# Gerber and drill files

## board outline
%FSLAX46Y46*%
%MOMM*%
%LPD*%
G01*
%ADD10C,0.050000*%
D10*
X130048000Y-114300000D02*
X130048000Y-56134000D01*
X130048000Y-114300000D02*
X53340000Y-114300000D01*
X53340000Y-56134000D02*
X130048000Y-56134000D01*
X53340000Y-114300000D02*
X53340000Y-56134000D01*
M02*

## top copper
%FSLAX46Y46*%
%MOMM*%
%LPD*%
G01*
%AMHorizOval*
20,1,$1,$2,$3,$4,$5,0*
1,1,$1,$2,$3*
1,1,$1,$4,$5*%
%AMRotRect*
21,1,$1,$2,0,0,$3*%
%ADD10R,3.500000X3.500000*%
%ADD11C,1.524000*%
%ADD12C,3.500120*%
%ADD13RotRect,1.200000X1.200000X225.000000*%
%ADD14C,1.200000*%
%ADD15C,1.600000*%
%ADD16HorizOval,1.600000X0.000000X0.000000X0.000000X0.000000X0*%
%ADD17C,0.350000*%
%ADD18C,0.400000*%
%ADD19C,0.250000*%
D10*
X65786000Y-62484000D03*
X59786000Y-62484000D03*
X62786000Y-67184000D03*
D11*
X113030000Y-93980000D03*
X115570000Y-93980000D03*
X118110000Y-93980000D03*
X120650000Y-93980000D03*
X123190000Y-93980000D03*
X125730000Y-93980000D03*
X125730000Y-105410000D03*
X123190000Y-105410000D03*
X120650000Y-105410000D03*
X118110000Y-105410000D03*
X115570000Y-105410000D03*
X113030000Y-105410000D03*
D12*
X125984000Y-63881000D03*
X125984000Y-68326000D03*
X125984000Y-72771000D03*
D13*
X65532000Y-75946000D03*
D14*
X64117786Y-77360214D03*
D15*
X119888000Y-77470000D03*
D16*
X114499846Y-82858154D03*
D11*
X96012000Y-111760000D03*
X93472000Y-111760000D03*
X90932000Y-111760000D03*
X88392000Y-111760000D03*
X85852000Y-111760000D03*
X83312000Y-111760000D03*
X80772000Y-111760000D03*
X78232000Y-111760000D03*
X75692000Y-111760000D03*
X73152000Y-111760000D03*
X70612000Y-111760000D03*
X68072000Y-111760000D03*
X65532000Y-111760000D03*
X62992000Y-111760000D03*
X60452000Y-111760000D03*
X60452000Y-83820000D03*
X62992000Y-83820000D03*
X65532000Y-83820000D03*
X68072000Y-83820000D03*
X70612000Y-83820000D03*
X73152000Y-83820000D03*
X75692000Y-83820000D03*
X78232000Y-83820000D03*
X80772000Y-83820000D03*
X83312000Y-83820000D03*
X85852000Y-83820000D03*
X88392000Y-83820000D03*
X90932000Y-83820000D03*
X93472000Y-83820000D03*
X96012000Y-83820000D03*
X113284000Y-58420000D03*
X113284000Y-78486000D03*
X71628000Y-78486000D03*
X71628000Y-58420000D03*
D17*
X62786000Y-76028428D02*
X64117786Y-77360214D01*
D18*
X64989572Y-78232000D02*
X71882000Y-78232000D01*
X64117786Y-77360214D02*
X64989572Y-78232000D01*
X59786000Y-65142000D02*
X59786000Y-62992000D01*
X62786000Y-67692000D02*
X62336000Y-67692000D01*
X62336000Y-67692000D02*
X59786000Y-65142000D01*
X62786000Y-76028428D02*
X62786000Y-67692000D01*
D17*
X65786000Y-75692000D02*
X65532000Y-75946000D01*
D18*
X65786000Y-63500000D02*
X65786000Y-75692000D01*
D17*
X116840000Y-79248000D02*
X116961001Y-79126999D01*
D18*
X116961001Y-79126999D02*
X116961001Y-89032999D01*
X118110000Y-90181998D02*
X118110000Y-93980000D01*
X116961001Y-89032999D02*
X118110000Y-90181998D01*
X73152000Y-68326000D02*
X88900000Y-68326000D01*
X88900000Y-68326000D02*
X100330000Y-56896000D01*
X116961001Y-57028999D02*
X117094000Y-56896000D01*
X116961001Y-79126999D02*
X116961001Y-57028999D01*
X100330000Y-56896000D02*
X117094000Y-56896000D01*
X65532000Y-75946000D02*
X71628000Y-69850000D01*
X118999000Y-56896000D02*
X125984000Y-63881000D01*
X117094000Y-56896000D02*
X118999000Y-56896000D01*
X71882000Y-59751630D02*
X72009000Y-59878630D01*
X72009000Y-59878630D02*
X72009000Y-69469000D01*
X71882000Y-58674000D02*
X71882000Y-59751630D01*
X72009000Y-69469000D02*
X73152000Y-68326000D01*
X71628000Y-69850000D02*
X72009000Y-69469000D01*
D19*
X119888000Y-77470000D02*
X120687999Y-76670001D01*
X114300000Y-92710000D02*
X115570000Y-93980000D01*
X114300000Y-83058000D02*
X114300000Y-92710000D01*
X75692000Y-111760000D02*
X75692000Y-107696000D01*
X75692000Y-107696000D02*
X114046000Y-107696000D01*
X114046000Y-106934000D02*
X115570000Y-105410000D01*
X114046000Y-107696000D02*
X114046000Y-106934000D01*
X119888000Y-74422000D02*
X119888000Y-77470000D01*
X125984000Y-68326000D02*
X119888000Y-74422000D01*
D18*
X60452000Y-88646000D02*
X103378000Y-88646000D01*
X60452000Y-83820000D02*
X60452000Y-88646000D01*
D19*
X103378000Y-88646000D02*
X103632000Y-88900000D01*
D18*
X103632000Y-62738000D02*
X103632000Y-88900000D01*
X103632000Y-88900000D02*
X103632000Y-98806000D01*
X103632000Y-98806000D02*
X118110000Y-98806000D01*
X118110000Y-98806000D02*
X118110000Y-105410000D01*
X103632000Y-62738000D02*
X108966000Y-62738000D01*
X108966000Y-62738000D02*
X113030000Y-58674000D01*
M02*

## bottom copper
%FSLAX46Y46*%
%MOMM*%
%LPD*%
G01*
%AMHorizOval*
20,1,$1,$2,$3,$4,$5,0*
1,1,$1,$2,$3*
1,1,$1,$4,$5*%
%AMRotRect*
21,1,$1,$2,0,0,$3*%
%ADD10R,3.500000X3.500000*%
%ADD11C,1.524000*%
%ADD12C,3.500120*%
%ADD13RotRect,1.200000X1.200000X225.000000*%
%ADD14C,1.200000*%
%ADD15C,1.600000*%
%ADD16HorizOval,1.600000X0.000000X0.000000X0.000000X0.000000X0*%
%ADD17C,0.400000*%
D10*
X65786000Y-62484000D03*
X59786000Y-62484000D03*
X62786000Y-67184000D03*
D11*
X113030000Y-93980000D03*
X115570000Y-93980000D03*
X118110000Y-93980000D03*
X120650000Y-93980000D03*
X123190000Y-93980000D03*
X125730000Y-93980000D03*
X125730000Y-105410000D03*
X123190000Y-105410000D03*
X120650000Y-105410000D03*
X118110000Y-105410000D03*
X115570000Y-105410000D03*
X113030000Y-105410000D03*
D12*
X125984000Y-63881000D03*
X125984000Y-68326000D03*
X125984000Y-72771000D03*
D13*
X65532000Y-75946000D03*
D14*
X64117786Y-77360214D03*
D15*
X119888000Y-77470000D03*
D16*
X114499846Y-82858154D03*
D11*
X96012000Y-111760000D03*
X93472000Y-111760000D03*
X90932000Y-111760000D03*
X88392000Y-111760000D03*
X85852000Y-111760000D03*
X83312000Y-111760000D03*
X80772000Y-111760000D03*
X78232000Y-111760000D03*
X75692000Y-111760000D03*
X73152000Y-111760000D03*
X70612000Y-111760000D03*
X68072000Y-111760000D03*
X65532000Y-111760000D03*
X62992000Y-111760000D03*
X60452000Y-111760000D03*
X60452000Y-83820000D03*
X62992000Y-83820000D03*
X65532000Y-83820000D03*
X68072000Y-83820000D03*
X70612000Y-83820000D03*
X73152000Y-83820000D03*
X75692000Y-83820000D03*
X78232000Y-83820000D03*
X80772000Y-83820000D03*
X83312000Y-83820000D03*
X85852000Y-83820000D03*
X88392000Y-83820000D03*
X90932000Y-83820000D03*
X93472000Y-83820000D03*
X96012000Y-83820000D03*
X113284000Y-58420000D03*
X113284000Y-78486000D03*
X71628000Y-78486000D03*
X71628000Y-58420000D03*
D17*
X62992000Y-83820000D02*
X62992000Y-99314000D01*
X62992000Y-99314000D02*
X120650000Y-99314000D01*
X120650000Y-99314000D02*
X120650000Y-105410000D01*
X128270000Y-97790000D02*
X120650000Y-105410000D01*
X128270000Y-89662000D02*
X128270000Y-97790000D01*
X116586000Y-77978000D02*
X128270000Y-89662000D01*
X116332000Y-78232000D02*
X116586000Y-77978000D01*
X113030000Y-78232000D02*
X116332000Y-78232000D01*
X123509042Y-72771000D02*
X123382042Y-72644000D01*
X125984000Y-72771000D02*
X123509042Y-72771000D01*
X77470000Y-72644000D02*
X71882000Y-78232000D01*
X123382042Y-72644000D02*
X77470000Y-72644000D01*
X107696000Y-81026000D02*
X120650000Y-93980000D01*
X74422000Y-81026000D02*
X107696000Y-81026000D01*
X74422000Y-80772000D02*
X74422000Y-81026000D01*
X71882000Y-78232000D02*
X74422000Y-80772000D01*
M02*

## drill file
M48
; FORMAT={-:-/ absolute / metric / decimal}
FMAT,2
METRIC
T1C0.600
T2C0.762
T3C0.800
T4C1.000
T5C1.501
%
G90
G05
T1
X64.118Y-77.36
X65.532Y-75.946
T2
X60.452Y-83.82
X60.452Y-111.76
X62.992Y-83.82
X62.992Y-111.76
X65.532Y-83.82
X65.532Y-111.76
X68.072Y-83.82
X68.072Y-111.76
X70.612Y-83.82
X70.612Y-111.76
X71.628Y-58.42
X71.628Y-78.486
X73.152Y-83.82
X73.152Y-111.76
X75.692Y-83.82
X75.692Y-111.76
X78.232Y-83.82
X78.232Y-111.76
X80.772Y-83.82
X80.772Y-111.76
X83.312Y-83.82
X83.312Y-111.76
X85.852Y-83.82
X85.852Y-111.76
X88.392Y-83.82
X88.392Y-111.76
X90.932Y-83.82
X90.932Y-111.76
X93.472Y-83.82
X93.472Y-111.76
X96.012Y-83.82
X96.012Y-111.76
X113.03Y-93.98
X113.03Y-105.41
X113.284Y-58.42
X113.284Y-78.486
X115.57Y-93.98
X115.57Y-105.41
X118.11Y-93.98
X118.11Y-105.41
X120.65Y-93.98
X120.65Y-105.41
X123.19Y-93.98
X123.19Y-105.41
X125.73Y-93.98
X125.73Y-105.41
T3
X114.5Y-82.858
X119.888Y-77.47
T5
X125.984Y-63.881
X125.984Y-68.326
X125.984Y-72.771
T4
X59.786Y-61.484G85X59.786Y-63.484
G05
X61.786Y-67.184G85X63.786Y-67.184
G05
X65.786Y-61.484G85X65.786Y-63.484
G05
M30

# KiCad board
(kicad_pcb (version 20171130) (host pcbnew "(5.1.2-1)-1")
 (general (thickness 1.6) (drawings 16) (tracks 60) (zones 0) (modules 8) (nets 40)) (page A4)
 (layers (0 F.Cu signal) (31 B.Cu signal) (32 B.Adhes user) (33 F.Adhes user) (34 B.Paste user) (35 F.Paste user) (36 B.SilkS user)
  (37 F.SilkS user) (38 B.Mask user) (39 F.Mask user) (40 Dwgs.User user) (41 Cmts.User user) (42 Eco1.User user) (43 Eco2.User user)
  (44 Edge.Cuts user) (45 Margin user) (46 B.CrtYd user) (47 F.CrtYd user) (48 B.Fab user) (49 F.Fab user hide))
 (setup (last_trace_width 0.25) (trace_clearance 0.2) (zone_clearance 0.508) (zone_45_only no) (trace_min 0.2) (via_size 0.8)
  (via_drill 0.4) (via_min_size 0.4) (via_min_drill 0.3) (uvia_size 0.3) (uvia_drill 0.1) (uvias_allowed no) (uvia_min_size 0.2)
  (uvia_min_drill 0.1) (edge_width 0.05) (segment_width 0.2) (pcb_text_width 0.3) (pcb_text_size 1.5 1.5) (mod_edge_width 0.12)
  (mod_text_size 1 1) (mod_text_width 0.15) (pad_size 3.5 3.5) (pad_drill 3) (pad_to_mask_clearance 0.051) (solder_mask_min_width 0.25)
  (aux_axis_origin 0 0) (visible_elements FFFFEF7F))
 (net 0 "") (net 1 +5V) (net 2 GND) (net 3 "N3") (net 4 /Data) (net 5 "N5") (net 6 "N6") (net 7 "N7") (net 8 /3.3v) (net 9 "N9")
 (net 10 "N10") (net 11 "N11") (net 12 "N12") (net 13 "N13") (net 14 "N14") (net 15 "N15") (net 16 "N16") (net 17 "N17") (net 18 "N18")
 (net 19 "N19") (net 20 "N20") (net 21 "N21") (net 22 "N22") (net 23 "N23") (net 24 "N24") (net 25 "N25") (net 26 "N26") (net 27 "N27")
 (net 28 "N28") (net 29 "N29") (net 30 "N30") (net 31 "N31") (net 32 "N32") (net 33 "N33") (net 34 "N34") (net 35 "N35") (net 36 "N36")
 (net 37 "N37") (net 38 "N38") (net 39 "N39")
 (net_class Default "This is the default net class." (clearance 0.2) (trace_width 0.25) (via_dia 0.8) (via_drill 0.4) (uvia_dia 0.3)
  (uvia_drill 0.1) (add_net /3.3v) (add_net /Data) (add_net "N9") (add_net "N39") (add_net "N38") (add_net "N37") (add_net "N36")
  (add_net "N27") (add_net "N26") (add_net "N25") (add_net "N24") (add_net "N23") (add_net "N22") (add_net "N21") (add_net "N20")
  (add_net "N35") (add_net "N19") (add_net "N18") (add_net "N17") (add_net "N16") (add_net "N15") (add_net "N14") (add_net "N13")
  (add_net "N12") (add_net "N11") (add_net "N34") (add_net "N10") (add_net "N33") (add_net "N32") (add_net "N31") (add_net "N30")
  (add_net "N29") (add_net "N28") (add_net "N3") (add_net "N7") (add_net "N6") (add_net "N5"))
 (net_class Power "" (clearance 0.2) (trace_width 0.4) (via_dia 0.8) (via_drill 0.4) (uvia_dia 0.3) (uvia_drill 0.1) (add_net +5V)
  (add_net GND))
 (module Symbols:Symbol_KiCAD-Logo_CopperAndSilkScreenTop (layer F.Cu) (at 119.126 88.392)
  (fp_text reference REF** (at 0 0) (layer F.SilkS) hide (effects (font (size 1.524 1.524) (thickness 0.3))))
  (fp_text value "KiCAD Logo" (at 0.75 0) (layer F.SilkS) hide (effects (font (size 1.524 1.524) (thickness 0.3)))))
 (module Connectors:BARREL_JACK (layer F.Cu) (at 65.786 62.484)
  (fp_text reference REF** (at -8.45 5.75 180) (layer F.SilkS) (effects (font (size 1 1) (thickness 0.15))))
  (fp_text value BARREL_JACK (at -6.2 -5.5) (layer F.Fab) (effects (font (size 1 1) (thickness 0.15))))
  (pad 1 thru_hole rect (at 0 0) (size 3.5 3.5) (drill oval 1 3) (layers *.Cu *.Mask) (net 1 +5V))
  (pad 2 thru_hole rect (at -6 0) (size 3.5 3.5) (drill oval 1 3) (layers *.Cu *.Mask) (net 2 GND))
  (pad 3 thru_hole rect (at -3 4.7) (size 3.5 3.5) (drill oval 3 1) (layers *.Cu *.Mask) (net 2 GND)))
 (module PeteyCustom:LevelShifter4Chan (layer F.Cu) (at 118.11 100.33 90)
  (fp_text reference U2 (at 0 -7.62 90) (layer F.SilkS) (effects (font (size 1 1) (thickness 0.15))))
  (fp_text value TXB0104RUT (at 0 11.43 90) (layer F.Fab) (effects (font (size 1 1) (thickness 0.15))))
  (pad 12 thru_hole circle (at 6.35 -5.08 90) (size 1.524 1.524) (drill 0.762) (layers *.Cu *.Mask) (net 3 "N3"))
  (pad 11 thru_hole circle (at 6.35 -2.54 90) (size 1.524 1.524) (drill 0.762) (layers *.Cu *.Mask) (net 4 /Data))
  (pad 10 thru_hole circle (at 6.35 0 90) (size 1.524 1.524) (drill 0.762) (layers *.Cu *.Mask) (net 1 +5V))
  (pad 9 thru_hole circle (at 6.35 2.54 90) (size 1.524 1.524) (drill 0.762) (layers *.Cu *.Mask) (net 2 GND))
  (pad 8 thru_hole circle (at 6.35 5.08 90) (size 1.524 1.524) (drill 0.762) (layers *.Cu *.Mask) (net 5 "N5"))
  (pad 7 thru_hole circle (at 6.35 7.62 90) (size 1.524 1.524) (drill 0.762) (layers *.Cu *.Mask) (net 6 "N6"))
  (pad 6 thru_hole circle (at -5.08 7.62 90) (size 1.524 1.524) (drill 0.762) (layers *.Cu *.Mask))
  (pad 5 thru_hole circle (at -5.08 5.08 90) (size 1.524 1.524) (drill 0.762) (layers *.Cu *.Mask) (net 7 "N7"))
  (pad 4 thru_hole circle (at -5.08 2.54 90) (size 1.524 1.524) (drill 0.762) (layers *.Cu *.Mask) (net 2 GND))
  (pad 3 thru_hole circle (at -5.08 0 90) (size 1.524 1.524) (drill 0.762) (layers *.Cu *.Mask) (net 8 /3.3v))
  (pad 2 thru_hole circle (at -5.08 -2.54 90) (size 1.524 1.524) (drill 0.762) (layers *.Cu *.Mask) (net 4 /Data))
  (pad 1 thru_hole circle (at -5.08 -5.08 90) (size 1.524 1.524) (drill 0.762) (layers *.Cu *.Mask)))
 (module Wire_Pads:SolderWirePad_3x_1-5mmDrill (layer F.Cu) (at 125.984 68.326 270)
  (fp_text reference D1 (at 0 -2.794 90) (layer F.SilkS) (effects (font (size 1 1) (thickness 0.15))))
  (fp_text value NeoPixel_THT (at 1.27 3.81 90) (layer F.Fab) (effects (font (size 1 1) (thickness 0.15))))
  (pad 1 thru_hole circle (at -4.445 0 270) (size 3.50012 3.50012) (drill 1.50114) (layers *.Cu *.Mask) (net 1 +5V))
  (pad 2 thru_hole circle (at 0 0 270) (size 3.50012 3.50012) (drill 1.50114) (layers *.Cu *.Mask) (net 4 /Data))
  (pad 3 thru_hole circle (at 4.445 0 270) (size 3.50012 3.50012) (drill 1.50114) (layers *.Cu *.Mask) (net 2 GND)))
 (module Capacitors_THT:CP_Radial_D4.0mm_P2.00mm (layer F.Cu) (at 65.532 75.946 225)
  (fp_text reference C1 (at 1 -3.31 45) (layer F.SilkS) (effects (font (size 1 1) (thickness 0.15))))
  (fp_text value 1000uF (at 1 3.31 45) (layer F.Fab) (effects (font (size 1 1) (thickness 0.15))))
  (pad 1 thru_hole rect (at 0 0 225) (size 1.2 1.2) (drill 0.6) (layers *.Cu *.Mask) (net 1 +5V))
  (pad 2 thru_hole circle (at 2 0 225) (size 1.2 1.2) (drill 0.6) (layers *.Cu *.Mask) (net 2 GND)))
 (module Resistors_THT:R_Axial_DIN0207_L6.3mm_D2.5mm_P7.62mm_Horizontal (layer F.Cu) (at 119.888 77.47 225)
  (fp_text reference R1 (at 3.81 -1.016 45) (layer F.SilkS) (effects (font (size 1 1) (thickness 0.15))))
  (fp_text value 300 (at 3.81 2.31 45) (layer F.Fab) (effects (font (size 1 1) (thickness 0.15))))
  (pad 1 thru_hole circle (at 0 0 225) (size 1.6 1.6) (drill 0.8) (layers *.Cu *.Mask) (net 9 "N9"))
  (pad 2 thru_hole oval (at 7.62 0 225) (size 1.6 1.6) (drill 0.8) (layers *.Cu *.Mask) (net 4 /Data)))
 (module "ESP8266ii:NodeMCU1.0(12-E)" (layer F.Cu) (at 78.232 97.79 270)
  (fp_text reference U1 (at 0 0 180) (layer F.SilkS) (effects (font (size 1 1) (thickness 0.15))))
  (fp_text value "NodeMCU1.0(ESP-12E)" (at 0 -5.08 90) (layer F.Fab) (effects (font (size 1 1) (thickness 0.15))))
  (pad 30 thru_hole circle (at 13.97 -17.78 270) (size 1.524 1.524) (drill 0.762) (layers *.Cu *.Mask F.SilkS) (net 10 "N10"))
  (pad 29 thru_hole circle (at 13.97 -15.24 270) (size 1.524 1.524) (drill 0.762) (layers *.Cu *.Mask F.SilkS) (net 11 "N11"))
  (pad 28 thru_hole circle (at 13.97 -12.7 270) (size 1.524 1.524) (drill 0.762) (layers *.Cu *.Mask F.SilkS) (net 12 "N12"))
  (pad 27 thru_hole circle (at 13.97 -10.16 270) (size 1.524 1.524) (drill 0.762) (layers *.Cu *.Mask F.SilkS) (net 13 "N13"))
  (pad 26 thru_hole circle (at 13.97 -7.62 270) (size 1.524 1.524) (drill 0.762) (layers *.Cu *.Mask F.SilkS) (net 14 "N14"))
  (pad 25 thru_hole circle (at 13.97 -5.08 270) (size 1.524 1.524) (drill 0.762) (layers *.Cu *.Mask F.SilkS) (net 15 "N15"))
  (pad 24 thru_hole circle (at 13.97 -2.54 270) (size 1.524 1.524) (drill 0.762) (layers *.Cu *.Mask F.SilkS) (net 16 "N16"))
  (pad 23 thru_hole circle (at 13.97 0 270) (size 1.524 1.524) (drill 0.762) (layers *.Cu *.Mask F.SilkS) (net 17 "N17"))
  (pad 22 thru_hole circle (at 13.97 2.54 270) (size 1.524 1.524) (drill 0.762) (layers *.Cu *.Mask F.SilkS) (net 4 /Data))
  (pad 21 thru_hole circle (at 13.97 5.08 270) (size 1.524 1.524) (drill 0.762) (layers *.Cu *.Mask F.SilkS) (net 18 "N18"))
  (pad 20 thru_hole circle (at 13.97 7.62 270) (size 1.524 1.524) (drill 0.762) (layers *.Cu *.Mask F.SilkS) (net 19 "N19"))
  (pad 19 thru_hole circle (at 13.97 10.16 270) (size 1.524 1.524) (drill 0.762) (layers *.Cu *.Mask F.SilkS) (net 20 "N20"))
  (pad 18 thru_hole circle (at 13.97 12.7 270) (size 1.524 1.524) (drill 0.762) (layers *.Cu *.Mask F.SilkS) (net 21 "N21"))
  (pad 17 thru_hole circle (at 13.97 15.24 270) (size 1.524 1.524) (drill 0.762) (layers *.Cu *.Mask F.SilkS) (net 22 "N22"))
  (pad 16 thru_hole circle (at 13.97 17.78 270) (size 1.524 1.524) (drill 0.762) (layers *.Cu *.Mask F.SilkS) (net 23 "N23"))
  (pad 15 thru_hole circle (at -13.97 17.78 270) (size 1.524 1.524) (drill 0.762) (layers *.Cu *.Mask F.SilkS) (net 8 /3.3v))
  (pad 14 thru_hole circle (at -13.97 15.24 270) (size 1.524 1.524) (drill 0.762) (layers *.Cu *.Mask F.SilkS) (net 2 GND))
  (pad 13 thru_hole circle (at -13.97 12.7 270) (size 1.524 1.524) (drill 0.762) (layers *.Cu *.Mask F.SilkS) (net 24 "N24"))
  (pad 12 thru_hole circle (at -13.97 10.16 270) (size 1.524 1.524) (drill 0.762) (layers *.Cu *.Mask F.SilkS) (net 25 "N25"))
  (pad 11 thru_hole circle (at -13.97 7.62 270) (size 1.524 1.524) (drill 0.762) (layers *.Cu *.Mask F.SilkS) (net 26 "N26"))
  (pad 10 thru_hole circle (at -13.97 5.08 270) (size 1.524 1.524) (drill 0.762) (layers *.Cu *.Mask F.SilkS) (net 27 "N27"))
  (pad 9 thru_hole circle (at -13.97 2.54 270) (size 1.524 1.524) (drill 0.762) (layers *.Cu *.Mask F.SilkS) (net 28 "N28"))
  (pad 8 thru_hole circle (at -13.97 0 270) (size 1.524 1.524) (drill 0.762) (layers *.Cu *.Mask F.SilkS) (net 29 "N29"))
  (pad 7 thru_hole circle (at -13.97 -2.54 270) (size 1.524 1.524) (drill 0.762) (layers *.Cu *.Mask F.SilkS) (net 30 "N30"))
  (pad 6 thru_hole circle (at -13.97 -5.08 270) (size 1.524 1.524) (drill 0.762) (layers *.Cu *.Mask F.SilkS) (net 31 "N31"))
  (pad 5 thru_hole circle (at -13.97 -7.62 270) (size 1.524 1.524) (drill 0.762) (layers *.Cu *.Mask F.SilkS) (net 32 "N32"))
  (pad 4 thru_hole circle (at -13.97 -10.16 270) (size 1.524 1.524) (drill 0.762) (layers *.Cu *.Mask F.SilkS) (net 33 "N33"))
  (pad 3 thru_hole circle (at -13.97 -12.7 270) (size 1.524 1.524) (drill 0.762) (layers *.Cu *.Mask F.SilkS) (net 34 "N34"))
  (pad 2 thru_hole circle (at -13.97 -15.24 270) (size 1.524 1.524) (drill 0.762) (layers *.Cu *.Mask F.SilkS) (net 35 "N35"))
  (pad 1 thru_hole circle (at -13.97 -17.78 270) (size 1.524 1.524) (drill 0.762) (layers *.Cu *.Mask F.SilkS) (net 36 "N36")))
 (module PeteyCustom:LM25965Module (layer F.Cu) (at 83.566 61.468)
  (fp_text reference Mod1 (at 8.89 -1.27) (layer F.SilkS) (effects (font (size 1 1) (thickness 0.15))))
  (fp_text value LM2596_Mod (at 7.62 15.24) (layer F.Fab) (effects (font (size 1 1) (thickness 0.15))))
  (pad 4 thru_hole circle (at 29.718 -3.048) (size 1.524 1.524) (drill 0.762) (layers *.Cu *.Mask) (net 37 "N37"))
  (pad 3 thru_hole circle (at 29.718 17.018) (size 1.524 1.524) (drill 0.762) (layers *.Cu *.Mask) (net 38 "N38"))
  (pad 2 thru_hole circle (at -11.938 17.018) (size 1.524 1.524) (drill 0.762) (layers *.Cu *.Mask) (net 2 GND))
  (pad 1 thru_hole circle (at -11.938 -3.048) (size 1.524 1.524) (drill 0.762) (layers *.Cu *.Mask) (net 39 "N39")))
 (gr_line (start 130.048 114.3) (end 130.048 56.134) (layer Edge.Cuts) (width 0.05))
 (gr_line (start 130.048 114.3) (end 53.34 114.3) (layer Edge.Cuts) (width 0.05))
 (gr_line (start 53.34 56.134) (end 130.048 56.134) (layer Edge.Cuts) (width 0.05))
 (gr_line (start 53.34 114.3) (end 53.34 56.134) (layer Edge.Cuts) (width 0.05))
 (segment (start 62.786 76.028428) (end 64.117786 77.360214) (width 0.35) (layer F.Cu) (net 2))
 (segment (start 62.992 83.82) (end 62.992 99.314) (width 0.4) (layer B.Cu) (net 2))
 (segment (start 62.992 99.314) (end 120.65 99.314) (width 0.4) (layer B.Cu) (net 2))
 (segment (start 120.65 99.314) (end 120.65 105.41) (width 0.4) (layer B.Cu) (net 2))
 (segment (start 128.27 97.79) (end 120.65 105.41) (width 0.4) (layer B.Cu) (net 2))
 (segment (start 128.27 89.662) (end 128.27 97.79) (width 0.4) (layer B.Cu) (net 2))
 (segment (start 116.586 77.978) (end 128.27 89.662) (width 0.4) (layer B.Cu) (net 2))
 (segment (start 116.332 78.232) (end 116.586 77.978) (width 0.4) (layer B.Cu) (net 2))
 (segment (start 113.03 78.232) (end 116.332 78.232) (width 0.4) (layer B.Cu) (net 2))
 (segment (start 123.509042 72.771) (end 123.382042 72.644) (width 0.4) (layer B.Cu) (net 2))
 (segment (start 125.984 72.771) (end 123.509042 72.771) (width 0.4) (layer B.Cu) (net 2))
 (segment (start 77.47 72.644) (end 71.882 78.232) (width 0.4) (layer B.Cu) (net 2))
 (segment (start 123.382042 72.644) (end 77.47 72.644) (width 0.4) (layer B.Cu) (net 2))
 (segment (start 64.989572 78.232) (end 71.882 78.232) (width 0.4) (layer F.Cu) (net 2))
 (segment (start 64.117786 77.360214) (end 64.989572 78.232) (width 0.4) (layer F.Cu) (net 2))
 (segment (start 107.696 81.026) (end 120.65 93.98) (width 0.4) (layer B.Cu) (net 2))
 (segment (start 74.422 81.026) (end 107.696 81.026) (width 0.4) (layer B.Cu) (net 2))
 (segment (start 74.422 80.772) (end 74.422 81.026) (width 0.4) (layer B.Cu) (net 2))
 (segment (start 71.882 78.232) (end 74.422 80.772) (width 0.4) (layer B.Cu) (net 2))
 (segment (start 59.786 65.142) (end 59.786 62.992) (width 0.4) (layer F.Cu) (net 2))
 (segment (start 62.786 67.692) (end 62.336 67.692) (width 0.4) (layer F.Cu) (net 2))
 (segment (start 62.336 67.692) (end 59.786 65.142) (width 0.4) (layer F.Cu) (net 2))
 (segment (start 62.786 76.028428) (end 62.786 67.692) (width 0.4) (layer F.Cu) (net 2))
 (segment (start 65.786 75.692) (end 65.532 75.946) (width 0.35) (layer F.Cu) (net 1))
 (segment (start 65.786 63.5) (end 65.786 75.692) (width 0.4) (layer F.Cu) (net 1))
 (segment (start 116.84 79.248) (end 116.961001 79.126999) (width 0.35) (layer F.Cu) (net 1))
 (segment (start 116.961001 79.126999) (end 116.961001 89.032999) (width 0.4) (layer F.Cu) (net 1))
 (segment (start 118.11 90.181998) (end 118.11 93.98) (width 0.4) (layer F.Cu) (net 1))
 (segment (start 116.961001 89.032999) (end 118.11 90.181998) (width 0.4) (layer F.Cu) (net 1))
 (segment (start 73.152 68.326) (end 88.9 68.326) (width 0.4) (layer F.Cu) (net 1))
 (segment (start 88.9 68.326) (end 100.33 56.896) (width 0.4) (layer F.Cu) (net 1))
 (segment (start 116.961001 57.028999) (end 117.094 56.896) (width 0.4) (layer F.Cu) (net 1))
 (segment (start 116.961001 79.126999) (end 116.961001 57.028999) (width 0.4) (layer F.Cu) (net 1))
 (segment (start 100.33 56.896) (end 117.094 56.896) (width 0.4) (layer F.Cu) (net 1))
 (segment (start 65.532 75.946) (end 71.628 69.85) (width 0.4) (layer F.Cu) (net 1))
 (segment (start 118.999 56.896) (end 125.984 63.881) (width 0.4) (layer F.Cu) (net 1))
 (segment (start 117.094 56.896) (end 118.999 56.896) (width 0.4) (layer F.Cu) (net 1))
 (segment (start 71.882 59.75163) (end 72.009 59.87863) (width 0.4) (layer F.Cu) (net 1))
 (segment (start 72.009 59.87863) (end 72.009 69.469) (width 0.4) (layer F.Cu) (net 1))
 (segment (start 71.882 58.674) (end 71.882 59.75163) (width 0.4) (layer F.Cu) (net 1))
 (segment (start 72.009 69.469) (end 73.152 68.326) (width 0.4) (layer F.Cu) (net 1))
 (segment (start 71.628 69.85) (end 72.009 69.469) (width 0.4) (layer F.Cu) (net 1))
 (segment (start 119.888 77.47) (end 120.687999 76.670001) (width 0.25) (layer F.Cu) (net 4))
 (segment (start 114.3 92.71) (end 115.57 93.98) (width 0.25) (layer F.Cu) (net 4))
 (segment (start 114.3 83.058) (end 114.3 92.71) (width 0.25) (layer F.Cu) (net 4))
 (segment (start 75.692 111.76) (end 75.692 107.696) (width 0.25) (layer F.Cu) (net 4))
 (segment (start 75.692 107.696) (end 114.046 107.696) (width 0.25) (layer F.Cu) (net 4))
 (segment (start 114.046 106.934) (end 115.57 105.41) (width 0.25) (layer F.Cu) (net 4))
 (segment (start 114.046 107.696) (end 114.046 106.934) (width 0.25) (layer F.Cu) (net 4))
 (segment (start 119.888 74.422) (end 119.888 77.47) (width 0.25) (layer F.Cu) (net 4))
 (segment (start 125.984 68.326) (end 119.888 74.422) (width 0.25) (layer F.Cu) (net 4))
 (segment (start 60.452 88.646) (end 103.378 88.646) (width 0.4) (layer F.Cu) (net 8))
 (segment (start 60.452 83.82) (end 60.452 88.646) (width 0.4) (layer F.Cu) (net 8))
 (segment (start 103.378 88.646) (end 103.632 88.9) (width 0.25) (layer F.Cu) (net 8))
 (segment (start 103.632 62.738) (end 103.632 88.9) (width 0.4) (layer F.Cu) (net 8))
 (segment (start 103.632 88.9) (end 103.632 98.806) (width 0.4) (layer F.Cu) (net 8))
 (segment (start 103.632 98.806) (end 118.11 98.806) (width 0.4) (layer F.Cu) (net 8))
 (segment (start 118.11 98.806) (end 118.11 105.41) (width 0.4) (layer F.Cu) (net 8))
 (segment (start 103.632 62.738) (end 108.966 62.738) (width 0.4) (layer F.Cu) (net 8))
 (segment (start 108.966 62.738) (end 113.03 58.674) (width 0.4) (layer F.Cu) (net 8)))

